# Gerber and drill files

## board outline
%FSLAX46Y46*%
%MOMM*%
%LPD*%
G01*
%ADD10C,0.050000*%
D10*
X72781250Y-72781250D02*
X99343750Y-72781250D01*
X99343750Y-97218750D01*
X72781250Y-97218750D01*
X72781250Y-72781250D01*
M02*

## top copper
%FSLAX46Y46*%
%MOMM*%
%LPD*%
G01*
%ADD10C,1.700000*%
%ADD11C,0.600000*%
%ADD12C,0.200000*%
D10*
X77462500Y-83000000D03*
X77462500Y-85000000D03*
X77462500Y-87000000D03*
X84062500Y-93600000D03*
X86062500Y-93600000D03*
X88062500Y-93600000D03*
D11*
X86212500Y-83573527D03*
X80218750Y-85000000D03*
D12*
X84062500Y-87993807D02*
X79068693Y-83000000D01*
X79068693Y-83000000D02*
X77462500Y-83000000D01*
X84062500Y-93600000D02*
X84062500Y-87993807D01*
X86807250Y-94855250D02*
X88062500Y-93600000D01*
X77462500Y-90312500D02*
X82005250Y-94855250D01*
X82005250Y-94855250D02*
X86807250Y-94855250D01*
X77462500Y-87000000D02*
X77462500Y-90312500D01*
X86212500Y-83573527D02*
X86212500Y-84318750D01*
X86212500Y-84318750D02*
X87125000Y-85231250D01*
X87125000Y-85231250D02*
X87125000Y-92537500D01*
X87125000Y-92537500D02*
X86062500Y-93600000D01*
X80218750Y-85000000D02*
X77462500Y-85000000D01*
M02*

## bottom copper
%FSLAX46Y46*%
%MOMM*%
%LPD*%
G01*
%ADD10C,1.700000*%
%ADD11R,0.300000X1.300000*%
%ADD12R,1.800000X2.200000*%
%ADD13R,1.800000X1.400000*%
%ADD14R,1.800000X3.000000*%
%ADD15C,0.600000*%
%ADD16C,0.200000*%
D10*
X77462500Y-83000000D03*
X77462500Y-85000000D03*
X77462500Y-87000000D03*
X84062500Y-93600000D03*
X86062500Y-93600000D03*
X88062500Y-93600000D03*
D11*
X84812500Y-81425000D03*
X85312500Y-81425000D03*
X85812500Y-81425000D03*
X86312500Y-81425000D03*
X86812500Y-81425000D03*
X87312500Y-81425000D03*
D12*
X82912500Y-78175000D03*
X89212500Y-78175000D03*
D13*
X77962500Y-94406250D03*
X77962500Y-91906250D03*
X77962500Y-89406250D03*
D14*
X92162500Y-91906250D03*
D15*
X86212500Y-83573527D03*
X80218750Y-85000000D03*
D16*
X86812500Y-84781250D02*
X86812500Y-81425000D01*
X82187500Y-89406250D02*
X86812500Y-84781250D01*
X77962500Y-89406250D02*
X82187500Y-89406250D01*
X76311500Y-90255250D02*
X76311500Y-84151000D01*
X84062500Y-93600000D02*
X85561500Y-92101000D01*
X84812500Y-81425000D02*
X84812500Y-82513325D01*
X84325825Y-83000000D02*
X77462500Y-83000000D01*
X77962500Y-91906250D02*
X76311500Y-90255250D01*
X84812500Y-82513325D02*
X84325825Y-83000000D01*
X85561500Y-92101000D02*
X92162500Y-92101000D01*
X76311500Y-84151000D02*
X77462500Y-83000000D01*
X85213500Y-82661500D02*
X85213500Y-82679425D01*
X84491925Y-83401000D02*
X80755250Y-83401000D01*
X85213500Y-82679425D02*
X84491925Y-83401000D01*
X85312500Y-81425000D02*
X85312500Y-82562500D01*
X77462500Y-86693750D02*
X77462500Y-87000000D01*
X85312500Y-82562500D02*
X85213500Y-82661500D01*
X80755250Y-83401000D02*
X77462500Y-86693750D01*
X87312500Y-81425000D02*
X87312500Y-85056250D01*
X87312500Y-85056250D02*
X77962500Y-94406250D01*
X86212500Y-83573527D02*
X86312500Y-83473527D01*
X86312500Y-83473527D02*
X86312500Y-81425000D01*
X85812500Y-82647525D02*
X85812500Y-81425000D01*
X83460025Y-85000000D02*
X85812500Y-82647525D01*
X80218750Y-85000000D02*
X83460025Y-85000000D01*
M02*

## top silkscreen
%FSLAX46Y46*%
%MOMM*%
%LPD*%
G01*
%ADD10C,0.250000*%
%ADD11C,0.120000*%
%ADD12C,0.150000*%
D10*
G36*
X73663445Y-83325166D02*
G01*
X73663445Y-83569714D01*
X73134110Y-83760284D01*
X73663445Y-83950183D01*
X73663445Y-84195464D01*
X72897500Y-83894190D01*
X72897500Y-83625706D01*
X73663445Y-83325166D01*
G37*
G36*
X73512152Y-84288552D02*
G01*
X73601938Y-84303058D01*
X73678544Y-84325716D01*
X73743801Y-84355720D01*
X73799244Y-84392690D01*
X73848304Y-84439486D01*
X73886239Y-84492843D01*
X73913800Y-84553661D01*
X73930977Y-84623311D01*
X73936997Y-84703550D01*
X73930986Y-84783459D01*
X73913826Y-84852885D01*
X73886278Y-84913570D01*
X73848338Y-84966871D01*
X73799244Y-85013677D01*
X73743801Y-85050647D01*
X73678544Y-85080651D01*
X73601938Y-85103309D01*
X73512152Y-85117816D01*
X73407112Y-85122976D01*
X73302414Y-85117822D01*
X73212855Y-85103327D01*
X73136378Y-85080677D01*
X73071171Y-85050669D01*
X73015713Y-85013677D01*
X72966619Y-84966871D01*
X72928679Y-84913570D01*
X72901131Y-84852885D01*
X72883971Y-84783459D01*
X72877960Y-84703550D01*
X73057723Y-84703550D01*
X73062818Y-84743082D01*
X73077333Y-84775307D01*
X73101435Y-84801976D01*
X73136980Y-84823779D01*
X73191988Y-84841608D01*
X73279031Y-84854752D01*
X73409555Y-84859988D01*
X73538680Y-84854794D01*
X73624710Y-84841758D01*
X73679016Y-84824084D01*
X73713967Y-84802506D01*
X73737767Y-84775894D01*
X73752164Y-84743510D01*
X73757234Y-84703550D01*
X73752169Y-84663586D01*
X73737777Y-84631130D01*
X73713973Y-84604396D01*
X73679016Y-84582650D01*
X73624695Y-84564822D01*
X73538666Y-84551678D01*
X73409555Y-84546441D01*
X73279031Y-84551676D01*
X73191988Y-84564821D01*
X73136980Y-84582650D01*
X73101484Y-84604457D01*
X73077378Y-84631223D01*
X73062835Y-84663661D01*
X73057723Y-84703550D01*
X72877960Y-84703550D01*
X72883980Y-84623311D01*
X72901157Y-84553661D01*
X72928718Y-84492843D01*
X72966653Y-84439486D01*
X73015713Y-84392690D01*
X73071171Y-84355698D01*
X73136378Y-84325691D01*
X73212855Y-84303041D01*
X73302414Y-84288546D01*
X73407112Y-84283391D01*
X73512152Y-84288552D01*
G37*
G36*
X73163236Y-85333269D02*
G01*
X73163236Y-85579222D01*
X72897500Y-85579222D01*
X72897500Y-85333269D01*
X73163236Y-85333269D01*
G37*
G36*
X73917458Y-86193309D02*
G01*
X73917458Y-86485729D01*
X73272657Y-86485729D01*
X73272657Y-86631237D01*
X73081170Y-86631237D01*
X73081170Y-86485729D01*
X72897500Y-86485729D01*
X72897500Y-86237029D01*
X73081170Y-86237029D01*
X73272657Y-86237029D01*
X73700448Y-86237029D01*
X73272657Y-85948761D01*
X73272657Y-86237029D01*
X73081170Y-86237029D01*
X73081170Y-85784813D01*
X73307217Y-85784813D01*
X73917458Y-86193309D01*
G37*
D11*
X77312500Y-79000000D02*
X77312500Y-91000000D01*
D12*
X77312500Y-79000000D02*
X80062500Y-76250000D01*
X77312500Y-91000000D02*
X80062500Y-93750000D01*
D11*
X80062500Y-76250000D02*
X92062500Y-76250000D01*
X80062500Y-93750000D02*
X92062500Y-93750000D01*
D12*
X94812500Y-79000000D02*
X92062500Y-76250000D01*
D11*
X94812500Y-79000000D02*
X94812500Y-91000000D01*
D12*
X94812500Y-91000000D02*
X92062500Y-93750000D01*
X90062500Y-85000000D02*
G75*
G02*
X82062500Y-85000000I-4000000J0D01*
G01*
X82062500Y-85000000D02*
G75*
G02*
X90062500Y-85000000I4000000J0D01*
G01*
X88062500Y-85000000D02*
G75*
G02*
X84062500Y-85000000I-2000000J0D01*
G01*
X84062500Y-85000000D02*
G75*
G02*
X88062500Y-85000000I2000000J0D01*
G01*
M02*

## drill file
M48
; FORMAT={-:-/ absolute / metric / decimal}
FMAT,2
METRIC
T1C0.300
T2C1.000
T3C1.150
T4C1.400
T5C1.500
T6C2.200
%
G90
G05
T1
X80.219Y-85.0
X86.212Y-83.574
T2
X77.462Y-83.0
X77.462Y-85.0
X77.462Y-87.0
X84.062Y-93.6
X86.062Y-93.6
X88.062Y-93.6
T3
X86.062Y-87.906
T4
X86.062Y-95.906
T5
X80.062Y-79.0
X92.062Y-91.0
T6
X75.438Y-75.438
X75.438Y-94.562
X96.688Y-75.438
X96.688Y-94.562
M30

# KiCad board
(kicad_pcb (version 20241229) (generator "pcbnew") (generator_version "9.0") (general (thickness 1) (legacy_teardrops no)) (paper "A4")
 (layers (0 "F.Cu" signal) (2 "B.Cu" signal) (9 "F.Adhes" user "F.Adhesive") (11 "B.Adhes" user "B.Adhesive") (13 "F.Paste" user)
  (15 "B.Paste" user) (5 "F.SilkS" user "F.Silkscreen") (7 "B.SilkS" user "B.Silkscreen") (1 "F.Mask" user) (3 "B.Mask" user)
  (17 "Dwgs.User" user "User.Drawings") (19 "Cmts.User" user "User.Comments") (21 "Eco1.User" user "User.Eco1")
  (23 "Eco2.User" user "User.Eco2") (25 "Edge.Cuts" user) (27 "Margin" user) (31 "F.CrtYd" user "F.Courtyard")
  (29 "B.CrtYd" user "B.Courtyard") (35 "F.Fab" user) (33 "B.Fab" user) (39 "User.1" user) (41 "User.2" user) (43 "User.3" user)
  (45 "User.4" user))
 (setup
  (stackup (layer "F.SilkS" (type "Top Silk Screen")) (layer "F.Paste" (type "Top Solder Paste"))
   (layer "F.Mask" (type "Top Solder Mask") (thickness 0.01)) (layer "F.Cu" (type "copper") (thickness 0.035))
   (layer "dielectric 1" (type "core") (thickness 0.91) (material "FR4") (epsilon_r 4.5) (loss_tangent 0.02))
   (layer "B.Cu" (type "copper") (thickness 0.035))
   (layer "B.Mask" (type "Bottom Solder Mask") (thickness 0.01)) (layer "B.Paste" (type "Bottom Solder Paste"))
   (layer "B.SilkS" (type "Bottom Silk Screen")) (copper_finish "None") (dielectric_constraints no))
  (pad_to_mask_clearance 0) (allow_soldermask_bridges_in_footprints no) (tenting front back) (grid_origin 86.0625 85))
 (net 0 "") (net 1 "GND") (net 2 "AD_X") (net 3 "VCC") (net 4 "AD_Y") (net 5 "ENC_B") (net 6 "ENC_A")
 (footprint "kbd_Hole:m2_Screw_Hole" (layer "F.Cu") (at 96.6875 75.4375)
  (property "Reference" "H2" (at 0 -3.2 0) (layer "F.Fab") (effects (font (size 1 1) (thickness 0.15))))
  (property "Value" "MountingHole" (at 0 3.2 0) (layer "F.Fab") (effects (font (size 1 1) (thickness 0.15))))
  (pad "" np_thru_hole circle (at 0 0) (size 2.2 2.2) (drill 2.2) (layers "*.Cu" "*.Mask")))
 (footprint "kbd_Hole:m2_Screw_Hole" (layer "F.Cu") (at 96.6875 94.5625)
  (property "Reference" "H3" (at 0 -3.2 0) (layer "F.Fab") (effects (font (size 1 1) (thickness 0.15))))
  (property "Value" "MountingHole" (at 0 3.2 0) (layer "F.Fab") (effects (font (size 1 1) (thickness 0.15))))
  (pad "" np_thru_hole circle (at 0 0) (size 2.2 2.2) (drill 2.2) (layers "*.Cu" "*.Mask")))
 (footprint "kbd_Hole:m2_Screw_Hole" (layer "F.Cu") (at 75.4375 94.5625)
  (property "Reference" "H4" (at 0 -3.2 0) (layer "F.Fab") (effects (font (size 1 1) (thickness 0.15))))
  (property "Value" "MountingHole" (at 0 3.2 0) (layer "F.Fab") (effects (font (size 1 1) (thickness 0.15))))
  (pad "" np_thru_hole circle (at 0 0) (size 2.2 2.2) (drill 2.2) (layers "*.Cu" "*.Mask")))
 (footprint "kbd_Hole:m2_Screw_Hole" (layer "F.Cu") (at 75.4375 75.4375)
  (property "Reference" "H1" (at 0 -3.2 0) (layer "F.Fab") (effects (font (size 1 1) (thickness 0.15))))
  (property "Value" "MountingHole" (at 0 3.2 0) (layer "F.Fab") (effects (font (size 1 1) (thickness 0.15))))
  (pad "" np_thru_hole circle (at 0 0) (size 2.2 2.2) (drill 2.2) (layers "*.Cu" "*.Mask")))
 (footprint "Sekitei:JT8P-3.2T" (layer "F.Cu") (at 86.0625 85 180)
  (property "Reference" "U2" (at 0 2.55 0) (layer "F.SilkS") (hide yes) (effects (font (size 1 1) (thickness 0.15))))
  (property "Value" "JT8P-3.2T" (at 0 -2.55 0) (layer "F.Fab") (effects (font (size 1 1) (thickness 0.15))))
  (fp_line (start 8.75 6) (end 8.75 -6) (stroke (width 0.12) (type solid)) (layer "F.SilkS"))
  (fp_line (start 8.75 6) (end 6 8.75) (stroke (width 0.15) (type solid)) (layer "F.SilkS"))
  (fp_line (start 8.75 -6) (end 6 -8.75) (stroke (width 0.15) (type solid)) (layer "F.SilkS"))
  (fp_line (start 6 8.75) (end -6 8.75) (stroke (width 0.12) (type solid)) (layer "F.SilkS"))
  (fp_line (start 6 -8.75) (end -6 -8.75) (stroke (width 0.12) (type solid)) (layer "F.SilkS"))
  (fp_line (start -8.75 6) (end -6 8.75) (stroke (width 0.15) (type solid)) (layer "F.SilkS"))
  (fp_line (start -8.75 6) (end -8.75 -6) (stroke (width 0.12) (type solid)) (layer "F.SilkS"))
  (fp_line (start -8.75 -6) (end -6 -8.75) (stroke (width 0.15) (type solid)) (layer "F.SilkS"))
  (fp_circle (center 0 0) (end 4 0) (stroke (width 0.15) (type solid)) (fill no) (layer "F.SilkS"))
  (fp_circle (center 0 0) (end 2 0) (stroke (width 0.15) (type solid)) (fill no) (layer "F.SilkS"))
  (pad "" np_thru_hole circle (at -6 -6 180) (size 1.5 1.5) (drill 1.5) (layers "*.Cu" "*.Mask"))
  (pad "" np_thru_hole circle (at 6 6 180) (size 1.5 1.5) (drill 1.5) (layers "*.Cu" "*.Mask"))
  (pad "1" thru_hole circle (at 8.6 2 180) (size 1.7 1.7) (drill 1) (layers "*.Cu" "*.Mask") (remove_unused_layers no) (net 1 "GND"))
  (pad "2" thru_hole circle (at 8.6 0 180) (size 1.7 1.7) (drill 1) (layers "*.Cu" "*.Mask") (remove_unused_layers no) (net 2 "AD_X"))
  (pad "3" thru_hole circle (at 8.6 -2 180) (size 1.7 1.7) (drill 1) (layers "*.Cu" "*.Mask") (remove_unused_layers no) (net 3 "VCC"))
  (pad "4" thru_hole circle (at 2 -8.6 180) (size 1.7 1.7) (drill 1) (layers "*.Cu" "*.Mask") (remove_unused_layers no) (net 1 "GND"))
  (pad "5" thru_hole circle (at 0 -8.6 180) (size 1.7 1.7) (drill 1) (layers "*.Cu" "*.Mask") (remove_unused_layers no) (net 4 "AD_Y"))
  (pad "6" thru_hole circle (at -2 -8.6 180) (size 1.7 1.7) (drill 1) (layers "*.Cu" "*.Mask") (remove_unused_layers no) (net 3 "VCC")))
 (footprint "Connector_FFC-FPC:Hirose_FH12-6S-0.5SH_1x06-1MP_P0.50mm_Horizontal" (layer "B.Cu") (at 86.0625 79.575)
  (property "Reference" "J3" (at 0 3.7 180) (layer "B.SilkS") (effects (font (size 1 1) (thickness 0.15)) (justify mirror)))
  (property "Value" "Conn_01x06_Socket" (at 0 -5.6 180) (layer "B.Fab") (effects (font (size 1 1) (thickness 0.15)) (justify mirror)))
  (pad "1" smd rect (at -1.25 1.85) (size 0.3 1.3) (layers "B.Cu" "B.Mask" "B.Paste") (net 1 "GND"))
  (pad "2" smd rect (at -0.75 1.85) (size 0.3 1.3) (layers "B.Cu" "B.Mask" "B.Paste") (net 3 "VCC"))
  (pad "3" smd rect (at -0.25 1.85) (size 0.3 1.3) (layers "B.Cu" "B.Mask" "B.Paste") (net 2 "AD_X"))
  (pad "4" smd rect (at 0.25 1.85) (size 0.3 1.3) (layers "B.Cu" "B.Mask" "B.Paste") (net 4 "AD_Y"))
  (pad "5" smd rect (at 0.75 1.85) (size 0.3 1.3) (layers "B.Cu" "B.Mask" "B.Paste") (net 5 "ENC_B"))
  (pad "6" smd rect (at 1.25 1.85) (size 0.3 1.3) (layers "B.Cu" "B.Mask" "B.Paste") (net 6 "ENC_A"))
  (pad "MP" smd rect (at -3.15 -1.4) (size 1.8 2.2) (layers "B.Cu" "B.Mask" "B.Paste"))
  (pad "MP" smd rect (at 3.15 -1.4) (size 1.8 2.2) (layers "B.Cu" "B.Mask" "B.Paste")))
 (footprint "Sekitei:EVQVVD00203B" (layer "B.Cu") (at 86.0875 91.90625 90)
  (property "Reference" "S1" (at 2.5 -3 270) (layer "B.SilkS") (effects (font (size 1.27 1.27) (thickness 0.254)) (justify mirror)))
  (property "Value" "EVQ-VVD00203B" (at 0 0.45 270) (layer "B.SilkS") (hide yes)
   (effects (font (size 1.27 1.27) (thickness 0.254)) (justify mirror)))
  (pad "" np_thru_hole circle (at -4 -0.025 90) (size 1.4 1.4) (drill 1.4) (layers "*.Cu" "*.Mask"))
  (pad "" np_thru_hole circle (at 4 -0.025 90) (size 1.15 1.15) (drill 1.15) (layers "*.Cu" "*.Mask"))
  (pad "1" smd rect (at -2.5 -8.125 90) (size 1.4 1.8) (layers "B.Cu" "B.Mask" "B.Paste") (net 6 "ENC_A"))
  (pad "2" smd rect (at 0 -8.125 90) (size 1.4 1.8) (layers "B.Cu" "B.Mask" "B.Paste") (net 1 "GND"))
  (pad "3" smd rect (at 2.5 -8.125 90) (size 1.4 1.8) (layers "B.Cu" "B.Mask" "B.Paste") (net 5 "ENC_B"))
  (pad "4" smd rect (at 0 6.075) (size 1.8 3) (layers "B.Cu" "B.Mask" "B.Paste") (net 1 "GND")))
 (gr_rect (start 72.78125 72.78125) (end 99.34375 97.21875) (stroke (width 0.05) (type default)) (fill no) (layer "Edge.Cuts"))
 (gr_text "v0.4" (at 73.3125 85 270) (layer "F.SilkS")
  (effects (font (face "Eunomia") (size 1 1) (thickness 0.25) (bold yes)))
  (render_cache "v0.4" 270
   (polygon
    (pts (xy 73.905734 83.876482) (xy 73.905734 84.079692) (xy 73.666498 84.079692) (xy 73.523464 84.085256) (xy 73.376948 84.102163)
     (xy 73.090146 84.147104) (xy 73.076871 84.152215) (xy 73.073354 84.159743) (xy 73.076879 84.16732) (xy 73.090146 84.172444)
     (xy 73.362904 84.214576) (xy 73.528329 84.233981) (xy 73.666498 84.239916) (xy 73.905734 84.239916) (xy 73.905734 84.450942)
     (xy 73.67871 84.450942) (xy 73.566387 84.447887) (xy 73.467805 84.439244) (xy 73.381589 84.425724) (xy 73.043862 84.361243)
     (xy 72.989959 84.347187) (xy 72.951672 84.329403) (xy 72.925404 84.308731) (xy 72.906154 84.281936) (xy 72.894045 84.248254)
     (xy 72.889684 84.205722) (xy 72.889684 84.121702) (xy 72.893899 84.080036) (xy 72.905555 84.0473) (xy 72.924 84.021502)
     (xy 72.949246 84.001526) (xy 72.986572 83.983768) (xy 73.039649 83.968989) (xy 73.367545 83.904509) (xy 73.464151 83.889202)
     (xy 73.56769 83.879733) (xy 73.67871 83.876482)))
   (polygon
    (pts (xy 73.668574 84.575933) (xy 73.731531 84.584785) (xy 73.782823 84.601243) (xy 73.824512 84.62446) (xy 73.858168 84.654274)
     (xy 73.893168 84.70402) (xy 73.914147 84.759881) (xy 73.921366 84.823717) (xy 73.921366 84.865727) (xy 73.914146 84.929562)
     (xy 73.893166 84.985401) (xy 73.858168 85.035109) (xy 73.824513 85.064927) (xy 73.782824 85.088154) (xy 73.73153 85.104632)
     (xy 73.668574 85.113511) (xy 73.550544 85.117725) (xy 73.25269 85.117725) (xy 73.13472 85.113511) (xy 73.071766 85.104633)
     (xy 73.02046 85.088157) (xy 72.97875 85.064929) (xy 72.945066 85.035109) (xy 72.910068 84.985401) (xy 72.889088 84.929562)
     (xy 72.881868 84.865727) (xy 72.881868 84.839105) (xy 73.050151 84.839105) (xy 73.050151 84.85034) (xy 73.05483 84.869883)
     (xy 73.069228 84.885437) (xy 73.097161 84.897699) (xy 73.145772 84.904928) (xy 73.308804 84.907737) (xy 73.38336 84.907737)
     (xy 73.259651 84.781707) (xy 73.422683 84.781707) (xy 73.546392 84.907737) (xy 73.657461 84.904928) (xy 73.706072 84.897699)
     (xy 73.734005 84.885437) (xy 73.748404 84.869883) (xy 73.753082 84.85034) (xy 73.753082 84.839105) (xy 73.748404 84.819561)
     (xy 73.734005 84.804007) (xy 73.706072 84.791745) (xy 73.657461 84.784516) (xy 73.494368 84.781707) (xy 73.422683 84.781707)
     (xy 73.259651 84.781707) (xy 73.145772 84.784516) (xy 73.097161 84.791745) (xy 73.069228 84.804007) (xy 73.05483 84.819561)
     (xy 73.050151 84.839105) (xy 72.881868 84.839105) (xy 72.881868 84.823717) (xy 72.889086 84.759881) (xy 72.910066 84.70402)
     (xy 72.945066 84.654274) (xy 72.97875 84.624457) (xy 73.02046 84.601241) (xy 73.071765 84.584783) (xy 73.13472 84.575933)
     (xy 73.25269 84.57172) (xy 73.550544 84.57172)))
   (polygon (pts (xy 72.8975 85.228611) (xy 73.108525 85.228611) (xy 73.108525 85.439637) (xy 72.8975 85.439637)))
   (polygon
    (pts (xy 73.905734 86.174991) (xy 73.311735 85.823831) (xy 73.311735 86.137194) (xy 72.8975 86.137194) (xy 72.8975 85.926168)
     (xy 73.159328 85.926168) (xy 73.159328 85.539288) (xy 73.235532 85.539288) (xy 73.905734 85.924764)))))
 (segment (start 86.8125 84.78125) (end 86.8125 81.425) (width 0.2) (layer "B.Cu") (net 5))
 (segment (start 82.1875 89.40625) (end 86.8125 84.78125) (width 0.2) (layer "B.Cu") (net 5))
 (segment (start 77.9625 89.40625) (end 82.1875 89.40625) (width 0.2) (layer "B.Cu") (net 5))
 (segment (start 84.0625 87.993807) (end 79.068693 83) (width 0.2) (layer "F.Cu") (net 1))
 (segment (start 79.068693 83) (end 77.4625 83) (width 0.2) (layer "F.Cu") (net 1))
 (segment (start 84.0625 93.6) (end 84.0625 87.993807) (width 0.2) (layer "F.Cu") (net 1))
 (segment (start 76.3115 90.25525) (end 76.3115 84.151) (width 0.2) (layer "B.Cu") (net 1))
 (segment (start 84.0625 93.6) (end 85.5615 92.101) (width 0.2) (layer "B.Cu") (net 1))
 (segment (start 84.8125 81.425) (end 84.8125 82.513325) (width 0.2) (layer "B.Cu") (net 1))
 (segment (start 84.325825 83) (end 77.4625 83) (width 0.2) (layer "B.Cu") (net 1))
 (segment (start 77.9625 91.90625) (end 76.3115 90.25525) (width 0.2) (layer "B.Cu") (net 1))
 (segment (start 84.8125 82.513325) (end 84.325825 83) (width 0.2) (layer "B.Cu") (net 1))
 (segment (start 85.5615 92.101) (end 92.1625 92.101) (width 0.2) (layer "B.Cu") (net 1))
 (segment (start 76.3115 84.151) (end 77.4625 83) (width 0.2) (layer "B.Cu") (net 1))
 (segment (start 86.80725 94.85525) (end 88.0625 93.6) (width 0.2) (layer "F.Cu") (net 3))
 (segment (start 77.4625 90.3125) (end 82.00525 94.85525) (width 0.2) (layer "F.Cu") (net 3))
 (segment (start 82.00525 94.85525) (end 86.80725 94.85525) (width 0.2) (layer "F.Cu") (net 3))
 (segment (start 77.4625 87) (end 77.4625 90.3125) (width 0.2) (layer "F.Cu") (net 3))
 (segment (start 85.2135 82.6615) (end 85.2135 82.679425) (width 0.2) (layer "B.Cu") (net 3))
 (segment (start 84.491925 83.401) (end 80.75525 83.401) (width 0.2) (layer "B.Cu") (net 3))
 (segment (start 85.2135 82.679425) (end 84.491925 83.401) (width 0.2) (layer "B.Cu") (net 3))
 (segment (start 85.3125 81.425) (end 85.3125 82.5625) (width 0.2) (layer "B.Cu") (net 3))
 (segment (start 77.4625 86.69375) (end 77.4625 87) (width 0.2) (layer "B.Cu") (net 3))
 (segment (start 85.3125 82.5625) (end 85.2135 82.6615) (width 0.2) (layer "B.Cu") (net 3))
 (segment (start 80.75525 83.401) (end 77.4625 86.69375) (width 0.2) (layer "B.Cu") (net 3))
 (segment (start 87.3125 81.425) (end 87.3125 85.05625) (width 0.2) (layer "B.Cu") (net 6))
 (segment (start 87.3125 85.05625) (end 77.9625 94.40625) (width 0.2) (layer "B.Cu") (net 6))
 (segment (start 86.2125 83.573527) (end 86.2125 84.31875) (width 0.2) (layer "F.Cu") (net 4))
 (segment (start 86.2125 84.31875) (end 87.125 85.23125) (width 0.2) (layer "F.Cu") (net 4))
 (segment (start 87.125 85.23125) (end 87.125 92.5375) (width 0.2) (layer "F.Cu") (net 4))
 (segment (start 87.125 92.5375) (end 86.0625 93.6) (width 0.2) (layer "F.Cu") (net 4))
 (via (at 86.2125 83.573527) (size 0.6) (drill 0.3) (layers "F.Cu" "B.Cu") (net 4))
 (segment (start 86.2125 83.573527) (end 86.3125 83.473527) (width 0.2) (layer "B.Cu") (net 4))
 (segment (start 86.3125 83.473527) (end 86.3125 81.425) (width 0.2) (layer "B.Cu") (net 4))
 (segment (start 80.21875 85) (end 77.4625 85) (width 0.2) (layer "F.Cu") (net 2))
 (via (at 80.21875 85) (size 0.6) (drill 0.3) (layers "F.Cu" "B.Cu") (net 2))
 (segment (start 85.8125 82.647525) (end 85.8125 81.425) (width 0.2) (layer "B.Cu") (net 2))
 (segment (start 83.460025 85) (end 85.8125 82.647525) (width 0.2) (layer "B.Cu") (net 2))
 (segment (start 80.21875 85) (end 83.460025 85) (width 0.2) (layer "B.Cu") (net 2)))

